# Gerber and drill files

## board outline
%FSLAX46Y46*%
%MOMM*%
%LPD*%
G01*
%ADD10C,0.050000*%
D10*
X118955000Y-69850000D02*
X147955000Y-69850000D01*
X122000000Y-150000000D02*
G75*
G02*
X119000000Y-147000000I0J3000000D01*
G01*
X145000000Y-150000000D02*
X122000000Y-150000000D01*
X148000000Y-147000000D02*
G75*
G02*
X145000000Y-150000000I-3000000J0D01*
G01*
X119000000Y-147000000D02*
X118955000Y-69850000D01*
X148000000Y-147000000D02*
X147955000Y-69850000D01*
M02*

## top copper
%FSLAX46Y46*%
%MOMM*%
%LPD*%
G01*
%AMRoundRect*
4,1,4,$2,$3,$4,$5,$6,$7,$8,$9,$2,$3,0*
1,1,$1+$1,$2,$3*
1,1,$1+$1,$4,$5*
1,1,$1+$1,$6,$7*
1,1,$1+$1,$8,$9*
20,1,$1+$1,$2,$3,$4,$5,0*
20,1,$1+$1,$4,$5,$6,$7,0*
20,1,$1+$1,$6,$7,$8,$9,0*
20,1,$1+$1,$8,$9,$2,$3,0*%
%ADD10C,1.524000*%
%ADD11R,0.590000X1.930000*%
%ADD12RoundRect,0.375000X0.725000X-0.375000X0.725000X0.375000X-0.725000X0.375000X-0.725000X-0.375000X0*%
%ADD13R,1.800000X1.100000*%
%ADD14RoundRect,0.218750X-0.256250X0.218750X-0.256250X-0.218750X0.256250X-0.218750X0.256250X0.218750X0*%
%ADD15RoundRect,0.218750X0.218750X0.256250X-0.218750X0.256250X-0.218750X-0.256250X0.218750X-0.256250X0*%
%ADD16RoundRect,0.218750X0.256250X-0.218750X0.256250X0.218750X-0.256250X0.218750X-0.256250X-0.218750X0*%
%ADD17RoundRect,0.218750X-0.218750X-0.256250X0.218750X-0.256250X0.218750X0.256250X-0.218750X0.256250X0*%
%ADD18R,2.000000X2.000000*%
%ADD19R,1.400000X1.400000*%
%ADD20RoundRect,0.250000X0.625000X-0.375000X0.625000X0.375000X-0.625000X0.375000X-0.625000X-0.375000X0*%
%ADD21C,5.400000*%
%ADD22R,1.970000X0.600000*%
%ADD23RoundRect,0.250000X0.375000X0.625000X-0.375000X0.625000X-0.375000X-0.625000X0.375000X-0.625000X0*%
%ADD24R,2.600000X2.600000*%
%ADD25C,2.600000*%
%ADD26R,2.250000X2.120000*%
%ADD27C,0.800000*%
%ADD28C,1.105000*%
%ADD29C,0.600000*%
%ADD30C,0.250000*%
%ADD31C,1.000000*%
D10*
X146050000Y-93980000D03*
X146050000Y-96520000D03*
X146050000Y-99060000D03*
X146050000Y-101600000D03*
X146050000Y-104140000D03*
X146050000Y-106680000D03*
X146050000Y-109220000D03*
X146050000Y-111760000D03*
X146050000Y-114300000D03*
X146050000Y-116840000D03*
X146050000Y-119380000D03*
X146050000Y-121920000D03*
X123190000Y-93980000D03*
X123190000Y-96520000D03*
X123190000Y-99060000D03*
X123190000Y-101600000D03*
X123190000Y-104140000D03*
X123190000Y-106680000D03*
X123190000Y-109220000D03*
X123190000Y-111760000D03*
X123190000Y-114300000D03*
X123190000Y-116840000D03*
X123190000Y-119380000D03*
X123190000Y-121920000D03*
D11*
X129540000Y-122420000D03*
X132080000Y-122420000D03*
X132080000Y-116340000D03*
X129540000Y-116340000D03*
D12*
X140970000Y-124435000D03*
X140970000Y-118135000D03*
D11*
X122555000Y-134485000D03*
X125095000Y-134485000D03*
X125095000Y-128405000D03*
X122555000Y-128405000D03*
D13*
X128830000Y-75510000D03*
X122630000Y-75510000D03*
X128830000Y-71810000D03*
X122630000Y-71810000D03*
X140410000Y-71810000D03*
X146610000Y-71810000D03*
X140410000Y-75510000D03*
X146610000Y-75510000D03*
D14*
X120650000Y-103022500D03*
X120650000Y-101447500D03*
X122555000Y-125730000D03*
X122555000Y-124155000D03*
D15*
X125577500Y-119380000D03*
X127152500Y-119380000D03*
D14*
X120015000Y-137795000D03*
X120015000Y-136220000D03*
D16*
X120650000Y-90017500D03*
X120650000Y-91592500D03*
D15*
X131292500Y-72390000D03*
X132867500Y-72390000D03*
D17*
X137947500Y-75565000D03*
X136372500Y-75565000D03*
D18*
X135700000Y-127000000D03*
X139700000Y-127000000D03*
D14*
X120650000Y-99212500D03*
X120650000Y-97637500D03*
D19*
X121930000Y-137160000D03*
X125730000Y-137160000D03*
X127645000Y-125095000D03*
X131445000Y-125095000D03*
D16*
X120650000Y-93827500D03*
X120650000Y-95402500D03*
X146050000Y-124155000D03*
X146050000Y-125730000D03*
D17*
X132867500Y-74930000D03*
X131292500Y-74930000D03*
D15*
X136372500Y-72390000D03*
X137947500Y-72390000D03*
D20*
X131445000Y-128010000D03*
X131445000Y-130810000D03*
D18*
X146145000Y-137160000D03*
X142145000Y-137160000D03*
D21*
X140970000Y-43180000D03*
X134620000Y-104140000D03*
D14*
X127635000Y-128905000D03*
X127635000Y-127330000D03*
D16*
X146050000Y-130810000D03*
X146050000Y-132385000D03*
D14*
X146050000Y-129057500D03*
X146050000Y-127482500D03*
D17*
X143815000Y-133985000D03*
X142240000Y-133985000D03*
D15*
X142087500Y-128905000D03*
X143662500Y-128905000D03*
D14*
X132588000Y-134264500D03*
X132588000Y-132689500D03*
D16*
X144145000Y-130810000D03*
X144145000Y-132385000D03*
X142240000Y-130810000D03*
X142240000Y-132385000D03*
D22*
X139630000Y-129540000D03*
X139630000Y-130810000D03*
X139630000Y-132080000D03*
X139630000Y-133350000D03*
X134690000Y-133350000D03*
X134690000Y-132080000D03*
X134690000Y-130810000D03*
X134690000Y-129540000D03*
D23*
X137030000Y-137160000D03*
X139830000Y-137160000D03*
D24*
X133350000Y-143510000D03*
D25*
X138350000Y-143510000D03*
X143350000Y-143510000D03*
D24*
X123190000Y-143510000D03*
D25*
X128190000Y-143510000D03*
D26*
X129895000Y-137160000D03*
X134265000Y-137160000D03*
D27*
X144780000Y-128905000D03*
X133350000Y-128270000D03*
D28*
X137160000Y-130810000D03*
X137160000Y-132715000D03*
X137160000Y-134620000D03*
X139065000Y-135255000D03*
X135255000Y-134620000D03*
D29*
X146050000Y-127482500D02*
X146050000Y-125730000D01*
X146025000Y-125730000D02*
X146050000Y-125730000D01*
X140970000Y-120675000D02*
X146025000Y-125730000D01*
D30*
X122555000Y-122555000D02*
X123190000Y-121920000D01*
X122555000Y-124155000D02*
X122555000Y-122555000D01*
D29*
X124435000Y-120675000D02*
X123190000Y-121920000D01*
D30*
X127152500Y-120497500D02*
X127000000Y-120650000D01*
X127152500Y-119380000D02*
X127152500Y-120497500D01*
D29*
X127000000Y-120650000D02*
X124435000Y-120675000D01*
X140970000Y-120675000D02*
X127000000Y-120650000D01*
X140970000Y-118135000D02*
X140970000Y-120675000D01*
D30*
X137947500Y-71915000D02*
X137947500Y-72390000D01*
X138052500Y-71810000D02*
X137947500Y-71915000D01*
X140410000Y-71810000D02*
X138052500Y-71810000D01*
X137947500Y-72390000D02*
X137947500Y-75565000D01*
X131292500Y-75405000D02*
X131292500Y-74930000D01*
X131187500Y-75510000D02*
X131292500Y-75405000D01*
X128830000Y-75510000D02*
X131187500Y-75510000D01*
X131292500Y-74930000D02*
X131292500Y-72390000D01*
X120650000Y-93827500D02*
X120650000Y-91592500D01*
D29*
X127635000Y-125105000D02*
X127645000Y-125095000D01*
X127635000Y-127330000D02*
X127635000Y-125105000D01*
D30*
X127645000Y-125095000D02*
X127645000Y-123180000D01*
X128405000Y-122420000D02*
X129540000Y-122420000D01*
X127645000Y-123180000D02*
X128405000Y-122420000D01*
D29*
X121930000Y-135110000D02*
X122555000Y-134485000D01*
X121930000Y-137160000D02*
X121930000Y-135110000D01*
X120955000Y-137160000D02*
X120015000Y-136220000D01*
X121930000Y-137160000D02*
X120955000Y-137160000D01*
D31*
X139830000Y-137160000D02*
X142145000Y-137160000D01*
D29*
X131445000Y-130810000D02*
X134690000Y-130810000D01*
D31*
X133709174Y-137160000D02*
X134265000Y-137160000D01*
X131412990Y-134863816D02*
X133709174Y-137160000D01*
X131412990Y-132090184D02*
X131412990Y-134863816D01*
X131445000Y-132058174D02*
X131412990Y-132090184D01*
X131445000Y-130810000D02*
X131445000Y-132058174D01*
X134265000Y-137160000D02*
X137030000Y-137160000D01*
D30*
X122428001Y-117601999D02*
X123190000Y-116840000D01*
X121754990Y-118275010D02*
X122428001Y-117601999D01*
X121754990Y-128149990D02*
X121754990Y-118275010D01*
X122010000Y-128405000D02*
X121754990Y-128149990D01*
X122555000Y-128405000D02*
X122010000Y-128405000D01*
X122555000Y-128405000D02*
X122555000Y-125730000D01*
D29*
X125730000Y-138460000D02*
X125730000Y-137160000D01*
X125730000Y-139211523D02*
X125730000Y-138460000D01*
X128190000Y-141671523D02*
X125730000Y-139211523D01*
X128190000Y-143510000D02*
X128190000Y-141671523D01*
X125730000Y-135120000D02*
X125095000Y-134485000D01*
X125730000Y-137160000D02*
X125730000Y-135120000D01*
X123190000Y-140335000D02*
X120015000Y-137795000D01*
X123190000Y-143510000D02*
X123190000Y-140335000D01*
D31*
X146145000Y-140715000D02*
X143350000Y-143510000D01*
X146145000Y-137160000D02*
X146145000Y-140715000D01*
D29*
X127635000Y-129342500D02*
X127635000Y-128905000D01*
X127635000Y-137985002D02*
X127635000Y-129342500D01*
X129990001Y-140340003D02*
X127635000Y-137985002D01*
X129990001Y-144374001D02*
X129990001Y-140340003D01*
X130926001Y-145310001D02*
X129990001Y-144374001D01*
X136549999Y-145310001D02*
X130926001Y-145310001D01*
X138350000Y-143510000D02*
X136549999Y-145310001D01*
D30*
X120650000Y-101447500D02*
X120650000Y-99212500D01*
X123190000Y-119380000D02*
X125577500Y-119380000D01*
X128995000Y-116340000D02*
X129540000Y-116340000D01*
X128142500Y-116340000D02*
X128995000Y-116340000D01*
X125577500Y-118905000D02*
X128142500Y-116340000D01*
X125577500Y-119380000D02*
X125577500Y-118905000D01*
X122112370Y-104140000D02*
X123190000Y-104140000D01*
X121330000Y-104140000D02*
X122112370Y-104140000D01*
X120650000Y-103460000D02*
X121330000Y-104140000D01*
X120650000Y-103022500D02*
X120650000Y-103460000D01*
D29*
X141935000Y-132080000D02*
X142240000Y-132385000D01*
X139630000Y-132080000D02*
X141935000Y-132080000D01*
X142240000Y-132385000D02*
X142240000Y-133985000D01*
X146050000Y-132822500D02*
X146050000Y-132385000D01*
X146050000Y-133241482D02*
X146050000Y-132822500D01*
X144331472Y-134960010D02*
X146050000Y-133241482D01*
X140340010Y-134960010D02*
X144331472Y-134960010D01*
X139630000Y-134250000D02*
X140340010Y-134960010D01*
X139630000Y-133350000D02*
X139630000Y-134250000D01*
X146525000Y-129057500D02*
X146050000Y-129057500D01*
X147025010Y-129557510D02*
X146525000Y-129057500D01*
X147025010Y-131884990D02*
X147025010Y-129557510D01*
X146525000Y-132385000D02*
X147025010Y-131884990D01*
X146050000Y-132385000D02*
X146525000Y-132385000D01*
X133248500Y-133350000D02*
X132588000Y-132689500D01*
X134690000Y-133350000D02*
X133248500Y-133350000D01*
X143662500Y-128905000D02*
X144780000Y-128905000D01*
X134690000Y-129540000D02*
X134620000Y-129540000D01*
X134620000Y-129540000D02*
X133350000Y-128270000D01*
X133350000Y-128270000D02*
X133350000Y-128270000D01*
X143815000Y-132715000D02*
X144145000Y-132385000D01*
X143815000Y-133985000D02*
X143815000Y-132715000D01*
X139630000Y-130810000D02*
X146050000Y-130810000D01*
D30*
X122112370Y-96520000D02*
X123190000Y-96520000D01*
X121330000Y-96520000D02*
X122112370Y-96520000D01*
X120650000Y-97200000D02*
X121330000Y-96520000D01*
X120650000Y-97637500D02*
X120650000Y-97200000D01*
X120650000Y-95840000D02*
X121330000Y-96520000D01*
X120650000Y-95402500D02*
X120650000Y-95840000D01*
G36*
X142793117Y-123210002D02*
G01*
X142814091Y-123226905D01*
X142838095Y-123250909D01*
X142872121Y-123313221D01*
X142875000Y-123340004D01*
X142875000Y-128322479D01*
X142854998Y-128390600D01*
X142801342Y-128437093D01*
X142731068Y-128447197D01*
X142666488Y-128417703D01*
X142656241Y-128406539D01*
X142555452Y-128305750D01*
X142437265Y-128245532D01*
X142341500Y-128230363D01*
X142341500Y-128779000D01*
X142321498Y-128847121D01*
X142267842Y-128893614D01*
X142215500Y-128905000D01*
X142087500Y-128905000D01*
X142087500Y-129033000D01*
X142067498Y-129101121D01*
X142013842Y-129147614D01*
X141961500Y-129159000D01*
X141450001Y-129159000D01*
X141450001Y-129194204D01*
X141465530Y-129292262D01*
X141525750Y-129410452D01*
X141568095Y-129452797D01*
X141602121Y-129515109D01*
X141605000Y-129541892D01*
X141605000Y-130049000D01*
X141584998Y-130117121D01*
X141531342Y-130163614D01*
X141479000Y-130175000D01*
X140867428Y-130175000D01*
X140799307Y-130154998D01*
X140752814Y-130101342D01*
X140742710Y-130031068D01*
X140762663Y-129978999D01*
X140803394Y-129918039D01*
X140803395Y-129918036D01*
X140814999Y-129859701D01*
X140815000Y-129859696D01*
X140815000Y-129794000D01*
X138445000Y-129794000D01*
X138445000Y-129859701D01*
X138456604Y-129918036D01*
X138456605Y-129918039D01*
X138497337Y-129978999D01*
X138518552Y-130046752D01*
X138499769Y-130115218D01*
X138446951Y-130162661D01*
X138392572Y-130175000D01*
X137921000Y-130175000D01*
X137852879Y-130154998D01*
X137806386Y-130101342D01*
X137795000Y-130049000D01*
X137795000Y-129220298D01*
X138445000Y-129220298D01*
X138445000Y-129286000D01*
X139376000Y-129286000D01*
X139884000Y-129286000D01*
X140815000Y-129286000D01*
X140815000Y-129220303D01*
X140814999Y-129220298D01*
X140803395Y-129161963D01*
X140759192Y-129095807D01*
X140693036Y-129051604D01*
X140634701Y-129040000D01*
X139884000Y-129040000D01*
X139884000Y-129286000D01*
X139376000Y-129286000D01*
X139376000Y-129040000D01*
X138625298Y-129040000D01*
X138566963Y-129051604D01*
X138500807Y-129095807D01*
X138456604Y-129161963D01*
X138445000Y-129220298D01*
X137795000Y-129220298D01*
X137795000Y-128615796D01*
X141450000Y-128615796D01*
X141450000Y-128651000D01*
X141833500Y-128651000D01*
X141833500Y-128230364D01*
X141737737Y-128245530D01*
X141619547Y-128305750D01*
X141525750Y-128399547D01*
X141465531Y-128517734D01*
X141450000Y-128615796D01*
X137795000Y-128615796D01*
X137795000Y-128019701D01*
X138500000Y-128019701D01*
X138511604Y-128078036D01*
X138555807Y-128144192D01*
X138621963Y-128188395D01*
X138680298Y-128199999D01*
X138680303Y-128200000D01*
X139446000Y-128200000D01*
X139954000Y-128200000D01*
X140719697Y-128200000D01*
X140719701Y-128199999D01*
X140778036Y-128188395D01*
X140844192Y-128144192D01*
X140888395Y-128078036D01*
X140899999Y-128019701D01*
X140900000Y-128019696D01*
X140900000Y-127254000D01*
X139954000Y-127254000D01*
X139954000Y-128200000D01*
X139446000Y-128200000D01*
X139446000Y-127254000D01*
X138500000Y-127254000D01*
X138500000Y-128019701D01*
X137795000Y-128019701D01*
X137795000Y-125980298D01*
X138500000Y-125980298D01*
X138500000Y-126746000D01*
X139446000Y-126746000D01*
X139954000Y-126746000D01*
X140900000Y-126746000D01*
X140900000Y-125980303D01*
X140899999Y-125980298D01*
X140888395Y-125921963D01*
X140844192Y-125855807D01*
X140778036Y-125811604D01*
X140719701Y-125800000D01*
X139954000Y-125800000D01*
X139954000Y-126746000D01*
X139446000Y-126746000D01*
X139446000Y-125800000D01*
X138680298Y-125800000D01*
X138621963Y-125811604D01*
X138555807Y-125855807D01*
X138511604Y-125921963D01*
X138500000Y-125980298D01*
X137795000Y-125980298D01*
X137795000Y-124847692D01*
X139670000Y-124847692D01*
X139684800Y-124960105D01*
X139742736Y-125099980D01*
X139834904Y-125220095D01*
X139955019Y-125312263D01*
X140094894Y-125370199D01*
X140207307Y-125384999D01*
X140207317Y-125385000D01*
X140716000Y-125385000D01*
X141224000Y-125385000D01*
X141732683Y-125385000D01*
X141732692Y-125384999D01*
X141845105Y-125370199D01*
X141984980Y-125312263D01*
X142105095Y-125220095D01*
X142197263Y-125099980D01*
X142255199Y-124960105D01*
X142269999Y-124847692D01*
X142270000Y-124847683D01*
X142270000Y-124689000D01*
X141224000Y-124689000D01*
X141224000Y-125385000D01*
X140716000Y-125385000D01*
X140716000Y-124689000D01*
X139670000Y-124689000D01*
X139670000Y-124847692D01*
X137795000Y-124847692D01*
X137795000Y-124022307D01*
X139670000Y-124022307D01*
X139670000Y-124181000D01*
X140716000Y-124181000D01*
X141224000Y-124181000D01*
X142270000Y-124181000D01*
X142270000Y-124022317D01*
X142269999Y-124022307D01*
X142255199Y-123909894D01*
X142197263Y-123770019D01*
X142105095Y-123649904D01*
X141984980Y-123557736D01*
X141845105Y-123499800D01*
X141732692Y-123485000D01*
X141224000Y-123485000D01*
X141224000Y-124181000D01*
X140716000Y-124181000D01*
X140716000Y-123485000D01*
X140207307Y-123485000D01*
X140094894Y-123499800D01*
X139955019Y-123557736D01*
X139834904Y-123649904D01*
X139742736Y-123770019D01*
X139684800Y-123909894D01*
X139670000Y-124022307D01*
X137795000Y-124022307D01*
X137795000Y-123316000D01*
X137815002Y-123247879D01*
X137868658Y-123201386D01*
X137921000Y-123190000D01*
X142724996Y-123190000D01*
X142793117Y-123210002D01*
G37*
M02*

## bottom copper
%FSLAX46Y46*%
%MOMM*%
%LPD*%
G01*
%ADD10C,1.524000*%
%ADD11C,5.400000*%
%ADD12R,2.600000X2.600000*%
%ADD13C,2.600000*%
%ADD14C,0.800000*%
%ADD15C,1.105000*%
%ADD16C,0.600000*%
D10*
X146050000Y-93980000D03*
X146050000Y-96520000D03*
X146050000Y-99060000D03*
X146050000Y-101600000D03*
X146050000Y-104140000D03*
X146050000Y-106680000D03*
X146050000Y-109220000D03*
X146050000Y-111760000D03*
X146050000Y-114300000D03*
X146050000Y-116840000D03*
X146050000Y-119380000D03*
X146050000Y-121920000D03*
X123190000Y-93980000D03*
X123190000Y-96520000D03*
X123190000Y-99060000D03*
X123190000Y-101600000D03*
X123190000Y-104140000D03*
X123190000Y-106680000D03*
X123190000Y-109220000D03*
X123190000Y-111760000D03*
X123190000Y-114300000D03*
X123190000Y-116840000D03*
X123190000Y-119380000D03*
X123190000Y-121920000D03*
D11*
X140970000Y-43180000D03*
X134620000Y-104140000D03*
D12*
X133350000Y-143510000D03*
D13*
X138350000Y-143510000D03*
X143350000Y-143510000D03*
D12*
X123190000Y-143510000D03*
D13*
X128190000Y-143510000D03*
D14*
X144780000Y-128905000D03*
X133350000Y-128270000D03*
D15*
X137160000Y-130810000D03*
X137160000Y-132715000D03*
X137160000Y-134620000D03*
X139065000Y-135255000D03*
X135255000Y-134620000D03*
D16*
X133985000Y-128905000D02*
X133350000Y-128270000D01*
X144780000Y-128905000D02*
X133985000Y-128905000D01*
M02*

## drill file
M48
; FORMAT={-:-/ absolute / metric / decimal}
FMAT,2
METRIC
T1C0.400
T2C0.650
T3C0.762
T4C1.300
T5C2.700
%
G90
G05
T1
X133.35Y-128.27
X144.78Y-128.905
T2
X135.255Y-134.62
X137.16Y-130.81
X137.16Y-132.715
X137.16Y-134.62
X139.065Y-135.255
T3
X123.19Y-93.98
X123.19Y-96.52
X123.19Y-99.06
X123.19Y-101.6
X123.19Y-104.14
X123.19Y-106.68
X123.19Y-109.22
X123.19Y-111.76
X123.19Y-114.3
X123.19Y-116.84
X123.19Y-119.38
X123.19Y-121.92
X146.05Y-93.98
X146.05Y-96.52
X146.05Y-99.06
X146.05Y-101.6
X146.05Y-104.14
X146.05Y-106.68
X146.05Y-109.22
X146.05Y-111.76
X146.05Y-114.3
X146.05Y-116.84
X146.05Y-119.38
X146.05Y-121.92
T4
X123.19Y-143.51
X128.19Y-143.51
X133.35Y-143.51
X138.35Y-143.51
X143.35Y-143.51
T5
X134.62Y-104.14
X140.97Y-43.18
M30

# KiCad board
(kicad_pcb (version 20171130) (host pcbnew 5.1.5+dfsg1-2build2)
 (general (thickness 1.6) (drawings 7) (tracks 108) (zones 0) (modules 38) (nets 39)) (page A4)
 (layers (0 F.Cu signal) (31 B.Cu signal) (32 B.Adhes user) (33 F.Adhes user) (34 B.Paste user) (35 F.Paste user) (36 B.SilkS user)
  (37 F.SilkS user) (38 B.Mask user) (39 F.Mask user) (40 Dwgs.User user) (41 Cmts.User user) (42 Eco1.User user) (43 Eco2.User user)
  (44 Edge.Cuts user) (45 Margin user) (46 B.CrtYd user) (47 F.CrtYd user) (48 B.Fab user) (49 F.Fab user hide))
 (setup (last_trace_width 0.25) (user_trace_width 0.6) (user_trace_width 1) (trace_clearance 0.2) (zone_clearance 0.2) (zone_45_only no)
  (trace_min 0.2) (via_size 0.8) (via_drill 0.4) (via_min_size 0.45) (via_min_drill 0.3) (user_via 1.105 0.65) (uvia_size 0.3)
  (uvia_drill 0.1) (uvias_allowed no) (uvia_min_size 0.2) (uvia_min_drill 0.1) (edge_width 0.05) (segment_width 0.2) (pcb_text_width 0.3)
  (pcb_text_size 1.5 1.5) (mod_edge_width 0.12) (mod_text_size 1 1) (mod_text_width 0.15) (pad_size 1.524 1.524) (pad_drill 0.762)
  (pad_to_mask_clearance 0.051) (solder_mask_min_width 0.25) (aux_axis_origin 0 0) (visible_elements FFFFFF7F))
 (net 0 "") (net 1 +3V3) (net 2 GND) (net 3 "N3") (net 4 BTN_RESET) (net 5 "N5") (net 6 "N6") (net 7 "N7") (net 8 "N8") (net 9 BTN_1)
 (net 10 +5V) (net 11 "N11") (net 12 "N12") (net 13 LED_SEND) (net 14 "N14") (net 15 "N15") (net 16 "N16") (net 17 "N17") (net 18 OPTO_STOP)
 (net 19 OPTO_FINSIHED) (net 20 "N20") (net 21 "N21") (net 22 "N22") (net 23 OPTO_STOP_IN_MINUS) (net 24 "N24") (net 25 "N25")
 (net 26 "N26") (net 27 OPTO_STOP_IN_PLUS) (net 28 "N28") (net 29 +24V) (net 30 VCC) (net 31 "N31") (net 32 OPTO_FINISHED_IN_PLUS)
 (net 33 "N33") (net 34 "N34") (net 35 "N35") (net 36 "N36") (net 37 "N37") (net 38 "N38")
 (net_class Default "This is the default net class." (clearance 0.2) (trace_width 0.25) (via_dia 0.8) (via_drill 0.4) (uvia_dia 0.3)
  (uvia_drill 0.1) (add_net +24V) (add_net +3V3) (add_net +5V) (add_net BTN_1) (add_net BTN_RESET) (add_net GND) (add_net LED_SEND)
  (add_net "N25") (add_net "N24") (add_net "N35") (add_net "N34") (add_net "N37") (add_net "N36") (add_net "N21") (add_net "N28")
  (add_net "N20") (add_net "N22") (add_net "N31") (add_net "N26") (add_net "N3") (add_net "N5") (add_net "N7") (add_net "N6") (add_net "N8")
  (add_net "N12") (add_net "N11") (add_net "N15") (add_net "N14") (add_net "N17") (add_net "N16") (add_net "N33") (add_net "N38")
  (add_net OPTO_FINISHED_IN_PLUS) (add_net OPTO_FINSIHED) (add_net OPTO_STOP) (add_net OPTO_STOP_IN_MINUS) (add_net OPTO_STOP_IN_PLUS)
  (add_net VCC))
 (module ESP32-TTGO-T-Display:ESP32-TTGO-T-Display (layer F.Cu) (at 134.62 104.14 180)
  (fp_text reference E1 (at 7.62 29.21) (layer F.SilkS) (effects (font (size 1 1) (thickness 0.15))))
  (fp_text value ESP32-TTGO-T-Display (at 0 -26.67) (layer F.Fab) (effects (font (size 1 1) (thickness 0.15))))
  (pad 3V3-1 thru_hole circle (at -11.43 10.16 180) (size 1.524 1.524) (drill 0.762) (layers *.Cu *.Mask) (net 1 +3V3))
  (pad G4 thru_hole circle (at -11.43 7.62 180) (size 1.524 1.524) (drill 0.762) (layers *.Cu *.Mask) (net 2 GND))
  (pad G3 thru_hole circle (at -11.43 5.08 180) (size 1.524 1.524) (drill 0.762) (layers *.Cu *.Mask) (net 2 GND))
  (pad 12 thru_hole circle (at -11.43 2.54 180) (size 1.524 1.524) (drill 0.762) (layers *.Cu *.Mask) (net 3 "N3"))
  (pad 13 thru_hole circle (at -11.43 0 180) (size 1.524 1.524) (drill 0.762) (layers *.Cu *.Mask) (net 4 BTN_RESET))
  (pad 15 thru_hole circle (at -11.43 -2.54 180) (size 1.524 1.524) (drill 0.762) (layers *.Cu *.Mask) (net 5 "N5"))
  (pad 2 thru_hole circle (at -11.43 -5.08 180) (size 1.524 1.524) (drill 0.762) (layers *.Cu *.Mask) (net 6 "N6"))
  (pad 17 thru_hole circle (at -11.43 -7.62 180) (size 1.524 1.524) (drill 0.762) (layers *.Cu *.Mask) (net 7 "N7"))
  (pad 22 thru_hole circle (at -11.43 -10.16 180) (size 1.524 1.524) (drill 0.762) (layers *.Cu *.Mask) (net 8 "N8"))
  (pad 21 thru_hole circle (at -11.43 -12.7 180) (size 1.524 1.524) (drill 0.762) (layers *.Cu *.Mask) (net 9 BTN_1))
  (pad G2 thru_hole circle (at -11.43 -15.24 180) (size 1.524 1.524) (drill 0.762) (layers *.Cu *.Mask) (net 2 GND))
  (pad G1 thru_hole circle (at -11.43 -17.78 180) (size 1.524 1.524) (drill 0.762) (layers *.Cu *.Mask) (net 2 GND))
  (pad 5V thru_hole circle (at 11.43 10.16 180) (size 1.524 1.524) (drill 0.762) (layers *.Cu *.Mask) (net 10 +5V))
  (pad G5 thru_hole circle (at 11.43 7.62 180) (size 1.524 1.524) (drill 0.762) (layers *.Cu *.Mask) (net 2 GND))
  (pad 27 thru_hole circle (at 11.43 5.08 180) (size 1.524 1.524) (drill 0.762) (layers *.Cu *.Mask) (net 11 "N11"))
  (pad 26 thru_hole circle (at 11.43 2.54 180) (size 1.524 1.524) (drill 0.762) (layers *.Cu *.Mask) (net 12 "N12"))
  (pad 25 thru_hole circle (at 11.43 0 180) (size 1.524 1.524) (drill 0.762) (layers *.Cu *.Mask) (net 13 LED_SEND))
  (pad 33 thru_hole circle (at 11.43 -2.54 180) (size 1.524 1.524) (drill 0.762) (layers *.Cu *.Mask) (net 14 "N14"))
  (pad 32 thru_hole circle (at 11.43 -5.08 180) (size 1.524 1.524) (drill 0.762) (layers *.Cu *.Mask) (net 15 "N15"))
  (pad 39 thru_hole circle (at 11.43 -7.62 180) (size 1.524 1.524) (drill 0.762) (layers *.Cu *.Mask) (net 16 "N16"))
  (pad 38 thru_hole circle (at 11.43 -10.16 180) (size 1.524 1.524) (drill 0.762) (layers *.Cu *.Mask) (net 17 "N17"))
  (pad 37 thru_hole circle (at 11.43 -12.7 180) (size 1.524 1.524) (drill 0.762) (layers *.Cu *.Mask) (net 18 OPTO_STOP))
  (pad 36 thru_hole circle (at 11.43 -15.24 180) (size 1.524 1.524) (drill 0.762) (layers *.Cu *.Mask) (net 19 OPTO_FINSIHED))
  (pad 3V3-2 thru_hole circle (at 11.43 -17.78 180) (size 1.524 1.524) (drill 0.762) (layers *.Cu *.Mask) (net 1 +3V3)))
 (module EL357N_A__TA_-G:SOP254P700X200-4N (layer F.Cu) (at 130.81 119.38 90)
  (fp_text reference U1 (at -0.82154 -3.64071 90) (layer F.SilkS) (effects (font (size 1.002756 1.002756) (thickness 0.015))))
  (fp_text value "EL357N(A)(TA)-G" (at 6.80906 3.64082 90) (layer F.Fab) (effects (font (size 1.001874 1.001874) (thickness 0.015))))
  (pad 1 smd rect (at -3.04 -1.27 90) (size 1.93 0.59) (layers F.Cu F.Paste F.Mask) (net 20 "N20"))
  (pad 2 smd rect (at -3.04 1.27 90) (size 1.93 0.59) (layers F.Cu F.Paste F.Mask) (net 2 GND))
  (pad 3 smd rect (at 3.04 1.27 90) (size 1.93 0.59) (layers F.Cu F.Paste F.Mask) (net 2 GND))
  (pad 4 smd rect (at 3.04 -1.27 90) (size 1.93 0.59) (layers F.Cu F.Paste F.Mask) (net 19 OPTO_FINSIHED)))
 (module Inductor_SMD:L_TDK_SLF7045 (layer F.Cu) (at 140.97 121.285 90)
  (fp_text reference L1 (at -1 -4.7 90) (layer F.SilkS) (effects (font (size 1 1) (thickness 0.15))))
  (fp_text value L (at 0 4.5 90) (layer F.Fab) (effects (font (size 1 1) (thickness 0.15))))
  (pad 1 smd roundrect (at -3.15 0 90) (size 1.5 2.2) (layers F.Cu F.Paste F.Mask) (roundrect_rratio 0.25) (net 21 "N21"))
  (pad 2 smd roundrect (at 3.15 0 90) (size 1.5 2.2) (layers F.Cu F.Paste F.Mask) (roundrect_rratio 0.25) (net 1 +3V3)))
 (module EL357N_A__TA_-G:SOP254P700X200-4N (layer F.Cu) (at 123.825 131.445 90)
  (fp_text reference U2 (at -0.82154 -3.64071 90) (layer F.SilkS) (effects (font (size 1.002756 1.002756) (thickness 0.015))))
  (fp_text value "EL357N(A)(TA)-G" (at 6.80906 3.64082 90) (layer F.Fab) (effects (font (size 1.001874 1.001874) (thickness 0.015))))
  (pad 1 smd rect (at -3.04 -1.27 90) (size 1.93 0.59) (layers F.Cu F.Paste F.Mask) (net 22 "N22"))
  (pad 2 smd rect (at -3.04 1.27 90) (size 1.93 0.59) (layers F.Cu F.Paste F.Mask) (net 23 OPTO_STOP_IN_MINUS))
  (pad 3 smd rect (at 3.04 1.27 90) (size 1.93 0.59) (layers F.Cu F.Paste F.Mask) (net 2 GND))
  (pad 4 smd rect (at 3.04 -1.27 90) (size 1.93 0.59) (layers F.Cu F.Paste F.Mask) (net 18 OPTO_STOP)))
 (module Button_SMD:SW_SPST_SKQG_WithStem (layer F.Cu) (at 125.73 73.66 180)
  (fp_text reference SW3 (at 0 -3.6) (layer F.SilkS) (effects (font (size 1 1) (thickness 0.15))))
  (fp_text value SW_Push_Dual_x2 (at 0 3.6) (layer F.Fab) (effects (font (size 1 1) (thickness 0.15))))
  (pad 1 smd rect (at -3.1 -1.85 180) (size 1.8 1.1) (layers F.Cu F.Paste F.Mask) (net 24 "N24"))
  (pad 1 smd rect (at 3.1 -1.85 180) (size 1.8 1.1) (layers F.Cu F.Paste F.Mask) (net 24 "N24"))
  (pad 2 smd rect (at -3.1 1.85 180) (size 1.8 1.1) (layers F.Cu F.Paste F.Mask) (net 2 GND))
  (pad 2 smd rect (at 3.1 1.85 180) (size 1.8 1.1) (layers F.Cu F.Paste F.Mask) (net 2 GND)))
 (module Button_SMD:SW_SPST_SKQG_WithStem (layer F.Cu) (at 143.51 73.66)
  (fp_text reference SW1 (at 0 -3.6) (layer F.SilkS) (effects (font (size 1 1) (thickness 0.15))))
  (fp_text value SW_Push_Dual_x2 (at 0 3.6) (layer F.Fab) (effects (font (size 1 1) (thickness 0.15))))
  (pad 1 smd rect (at -3.1 -1.85) (size 1.8 1.1) (layers F.Cu F.Paste F.Mask) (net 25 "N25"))
  (pad 1 smd rect (at 3.1 -1.85) (size 1.8 1.1) (layers F.Cu F.Paste F.Mask) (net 25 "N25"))
  (pad 2 smd rect (at -3.1 1.85) (size 1.8 1.1) (layers F.Cu F.Paste F.Mask) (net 2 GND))
  (pad 2 smd rect (at 3.1 1.85) (size 1.8 1.1) (layers F.Cu F.Paste F.Mask) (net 2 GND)))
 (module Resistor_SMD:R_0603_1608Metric (layer F.Cu) (at 120.65 102.235 270)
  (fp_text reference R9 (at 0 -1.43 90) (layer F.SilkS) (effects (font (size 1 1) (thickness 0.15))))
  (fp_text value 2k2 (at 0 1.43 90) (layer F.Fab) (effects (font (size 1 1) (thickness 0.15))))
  (pad 2 smd roundrect (at 0.7875 0 270) (size 0.875 0.95) (layers F.Cu F.Paste F.Mask) (roundrect_rratio 0.25) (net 13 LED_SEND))
  (pad 1 smd roundrect (at -0.7875 0 270) (size 0.875 0.95) (layers F.Cu F.Paste F.Mask) (roundrect_rratio 0.25) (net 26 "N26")))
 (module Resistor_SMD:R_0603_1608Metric (layer F.Cu) (at 122.555 124.9425 270)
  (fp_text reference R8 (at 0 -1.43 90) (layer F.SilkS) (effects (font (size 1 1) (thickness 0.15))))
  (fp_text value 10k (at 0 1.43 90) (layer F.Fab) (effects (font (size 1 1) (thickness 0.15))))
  (pad 2 smd roundrect (at 0.7875 0 270) (size 0.875 0.95) (layers F.Cu F.Paste F.Mask) (roundrect_rratio 0.25) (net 18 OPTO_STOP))
  (pad 1 smd roundrect (at -0.7875 0 270) (size 0.875 0.95) (layers F.Cu F.Paste F.Mask) (roundrect_rratio 0.25) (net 1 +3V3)))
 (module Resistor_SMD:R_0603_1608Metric (layer F.Cu) (at 126.365 119.38 180)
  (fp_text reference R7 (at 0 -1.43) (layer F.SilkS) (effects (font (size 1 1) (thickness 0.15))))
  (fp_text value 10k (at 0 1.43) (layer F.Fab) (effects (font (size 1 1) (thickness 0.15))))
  (pad 2 smd roundrect (at 0.7875 0 180) (size 0.875 0.95) (layers F.Cu F.Paste F.Mask) (roundrect_rratio 0.25) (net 19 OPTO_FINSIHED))
  (pad 1 smd roundrect (at -0.7875 0 180) (size 0.875 0.95) (layers F.Cu F.Paste F.Mask) (roundrect_rratio 0.25) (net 1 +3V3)))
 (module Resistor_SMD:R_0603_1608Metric (layer F.Cu) (at 120.015 137.0075 270)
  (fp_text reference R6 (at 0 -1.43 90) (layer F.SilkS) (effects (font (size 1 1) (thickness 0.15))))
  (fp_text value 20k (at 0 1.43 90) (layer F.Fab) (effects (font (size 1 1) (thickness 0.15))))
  (pad 2 smd roundrect (at 0.7875 0 270) (size 0.875 0.95) (layers F.Cu F.Paste F.Mask) (roundrect_rratio 0.25) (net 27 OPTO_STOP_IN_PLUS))
  (pad 1 smd roundrect (at -0.7875 0 270) (size 0.875 0.95) (layers F.Cu F.Paste F.Mask) (roundrect_rratio 0.25) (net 22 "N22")))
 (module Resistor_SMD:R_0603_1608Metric (layer F.Cu) (at 120.65 90.805 90)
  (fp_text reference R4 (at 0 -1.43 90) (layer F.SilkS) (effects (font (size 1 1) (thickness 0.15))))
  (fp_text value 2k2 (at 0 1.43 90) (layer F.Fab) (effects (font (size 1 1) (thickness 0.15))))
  (pad 2 smd roundrect (at 0.7875 0 90) (size 0.875 0.95) (layers F.Cu F.Paste F.Mask) (roundrect_rratio 0.25) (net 1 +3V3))
  (pad 1 smd roundrect (at -0.7875 0 90) (size 0.875 0.95) (layers F.Cu F.Paste F.Mask) (roundrect_rratio 0.25) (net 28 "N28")))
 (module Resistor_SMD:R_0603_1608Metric (layer F.Cu) (at 132.08 72.39 180)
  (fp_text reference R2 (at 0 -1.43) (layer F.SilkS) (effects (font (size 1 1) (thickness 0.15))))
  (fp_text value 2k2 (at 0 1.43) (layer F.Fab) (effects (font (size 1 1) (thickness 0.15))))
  (pad 2 smd roundrect (at 0.7875 0 180) (size 0.875 0.95) (layers F.Cu F.Paste F.Mask) (roundrect_rratio 0.25) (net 24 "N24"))
  (pad 1 smd roundrect (at -0.7875 0 180) (size 0.875 0.95) (layers F.Cu F.Paste F.Mask) (roundrect_rratio 0.25) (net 9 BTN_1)))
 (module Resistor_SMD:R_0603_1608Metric (layer F.Cu) (at 137.16 75.565)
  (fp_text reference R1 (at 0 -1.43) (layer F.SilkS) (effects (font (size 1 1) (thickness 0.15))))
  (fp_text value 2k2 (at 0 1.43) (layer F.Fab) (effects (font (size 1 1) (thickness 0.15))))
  (pad 2 smd roundrect (at 0.7875 0) (size 0.875 0.95) (layers F.Cu F.Paste F.Mask) (roundrect_rratio 0.25) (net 25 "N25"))
  (pad 1 smd roundrect (at -0.7875 0) (size 0.875 0.95) (layers F.Cu F.Paste F.Mask) (roundrect_rratio 0.25) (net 4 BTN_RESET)))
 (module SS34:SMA (layer F.Cu) (at 137.7 127 180)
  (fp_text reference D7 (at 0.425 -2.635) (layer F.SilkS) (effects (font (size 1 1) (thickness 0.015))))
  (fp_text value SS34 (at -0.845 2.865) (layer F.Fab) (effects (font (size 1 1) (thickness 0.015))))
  (pad A smd rect (at 2 0 180) (size 2 2) (layers F.Cu F.Paste F.Mask) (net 2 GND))
  (pad C smd rect (at -2 0 180) (size 2 2) (layers F.Cu F.Paste F.Mask) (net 21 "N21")))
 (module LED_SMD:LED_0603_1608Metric (layer F.Cu) (at 120.65 98.425 270)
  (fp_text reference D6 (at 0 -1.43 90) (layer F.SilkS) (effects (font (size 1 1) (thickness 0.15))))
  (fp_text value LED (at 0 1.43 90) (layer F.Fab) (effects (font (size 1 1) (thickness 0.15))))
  (pad 2 smd roundrect (at 0.7875 0 270) (size 0.875 0.95) (layers F.Cu F.Paste F.Mask) (roundrect_rratio 0.25) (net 26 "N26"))
  (pad 1 smd roundrect (at -0.7875 0 270) (size 0.875 0.95) (layers F.Cu F.Paste F.Mask) (roundrect_rratio 0.25) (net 2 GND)))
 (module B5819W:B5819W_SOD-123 (layer F.Cu) (at 123.83 137.16)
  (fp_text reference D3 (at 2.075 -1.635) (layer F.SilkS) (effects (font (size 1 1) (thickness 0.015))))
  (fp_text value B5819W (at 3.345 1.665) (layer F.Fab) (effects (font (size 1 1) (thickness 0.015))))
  (pad C smd rect (at -1.9 0) (size 1.4 1.4) (layers F.Cu F.Paste F.Mask) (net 22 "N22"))
  (pad A smd rect (at 1.9 0) (size 1.4 1.4) (layers F.Cu F.Paste F.Mask) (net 23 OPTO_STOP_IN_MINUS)))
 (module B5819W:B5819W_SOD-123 (layer F.Cu) (at 129.545 125.095)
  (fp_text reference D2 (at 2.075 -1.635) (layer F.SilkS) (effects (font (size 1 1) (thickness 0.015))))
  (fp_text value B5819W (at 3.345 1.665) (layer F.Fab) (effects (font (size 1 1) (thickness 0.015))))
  (pad C smd rect (at -1.9 0) (size 1.4 1.4) (layers F.Cu F.Paste F.Mask) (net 20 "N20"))
  (pad A smd rect (at 1.9 0) (size 1.4 1.4) (layers F.Cu F.Paste F.Mask) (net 2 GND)))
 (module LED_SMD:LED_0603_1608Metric (layer F.Cu) (at 120.65 94.615 90)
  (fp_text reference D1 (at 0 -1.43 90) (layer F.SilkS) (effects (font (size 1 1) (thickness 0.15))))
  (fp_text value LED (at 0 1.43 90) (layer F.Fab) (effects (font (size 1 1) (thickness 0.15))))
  (pad 2 smd roundrect (at 0.7875 0 90) (size 0.875 0.95) (layers F.Cu F.Paste F.Mask) (roundrect_rratio 0.25) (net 28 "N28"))
  (pad 1 smd roundrect (at -0.7875 0 90) (size 0.875 0.95) (layers F.Cu F.Paste F.Mask) (roundrect_rratio 0.25) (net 2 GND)))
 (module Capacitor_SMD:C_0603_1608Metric (layer F.Cu) (at 146.05 124.9425 90)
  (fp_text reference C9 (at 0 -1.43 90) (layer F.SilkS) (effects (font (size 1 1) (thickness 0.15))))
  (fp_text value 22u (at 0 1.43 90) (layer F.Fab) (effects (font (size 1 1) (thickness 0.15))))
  (pad 2 smd roundrect (at 0.7875 0 90) (size 0.875 0.95) (layers F.Cu F.Paste F.Mask) (roundrect_rratio 0.25) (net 2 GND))
  (pad 1 smd roundrect (at -0.7875 0 90) (size 0.875 0.95) (layers F.Cu F.Paste F.Mask) (roundrect_rratio 0.25) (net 1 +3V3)))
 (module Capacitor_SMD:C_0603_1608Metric (layer F.Cu) (at 132.08 74.93)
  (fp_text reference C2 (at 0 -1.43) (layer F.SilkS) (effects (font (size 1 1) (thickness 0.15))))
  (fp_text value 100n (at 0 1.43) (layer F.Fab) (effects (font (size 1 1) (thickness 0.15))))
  (pad 2 smd roundrect (at 0.7875 0) (size 0.875 0.95) (layers F.Cu F.Paste F.Mask) (roundrect_rratio 0.25) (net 2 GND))
  (pad 1 smd roundrect (at -0.7875 0) (size 0.875 0.95) (layers F.Cu F.Paste F.Mask) (roundrect_rratio 0.25) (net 24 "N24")))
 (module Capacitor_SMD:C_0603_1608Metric (layer F.Cu) (at 137.16 72.39 180)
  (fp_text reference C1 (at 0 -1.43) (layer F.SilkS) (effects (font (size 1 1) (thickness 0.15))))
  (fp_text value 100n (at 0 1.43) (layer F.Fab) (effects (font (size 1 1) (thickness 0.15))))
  (pad 2 smd roundrect (at 0.7875 0 180) (size 0.875 0.95) (layers F.Cu F.Paste F.Mask) (roundrect_rratio 0.25) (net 2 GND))
  (pad 1 smd roundrect (at -0.7875 0 180) (size 0.875 0.95) (layers F.Cu F.Paste F.Mask) (roundrect_rratio 0.25) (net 25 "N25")))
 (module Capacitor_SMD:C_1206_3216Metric (layer F.Cu) (at 131.445 129.41 90)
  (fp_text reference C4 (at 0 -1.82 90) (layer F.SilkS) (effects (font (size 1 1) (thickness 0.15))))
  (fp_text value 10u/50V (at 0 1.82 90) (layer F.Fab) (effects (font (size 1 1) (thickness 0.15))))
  (pad 2 smd roundrect (at 1.4 0 90) (size 1.25 1.75) (layers F.Cu F.Paste F.Mask) (roundrect_rratio 0.2) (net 2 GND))
  (pad 1 smd roundrect (at -1.4 0 90) (size 1.25 1.75) (layers F.Cu F.Paste F.Mask) (roundrect_rratio 0.2) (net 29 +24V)))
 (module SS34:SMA (layer F.Cu) (at 144.145 137.16)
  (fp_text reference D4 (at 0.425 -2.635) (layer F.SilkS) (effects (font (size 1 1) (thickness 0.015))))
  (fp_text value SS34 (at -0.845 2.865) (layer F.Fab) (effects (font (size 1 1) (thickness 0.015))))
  (pad A smd rect (at 2 0) (size 2 2) (layers F.Cu F.Paste F.Mask) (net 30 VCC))
  (pad C smd rect (at -2 0) (size 2 2) (layers F.Cu F.Paste F.Mask) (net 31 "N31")))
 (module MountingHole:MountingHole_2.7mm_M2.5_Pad (layer F.Cu) (at 140.97 43.18)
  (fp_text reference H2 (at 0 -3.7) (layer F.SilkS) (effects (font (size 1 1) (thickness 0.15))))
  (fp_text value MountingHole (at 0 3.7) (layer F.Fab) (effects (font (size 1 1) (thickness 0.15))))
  (pad 1 thru_hole circle (at 0 0) (size 5.4 5.4) (drill 2.7) (layers *.Cu *.Mask)))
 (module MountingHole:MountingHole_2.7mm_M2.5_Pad (layer F.Cu) (at 134.62 104.14)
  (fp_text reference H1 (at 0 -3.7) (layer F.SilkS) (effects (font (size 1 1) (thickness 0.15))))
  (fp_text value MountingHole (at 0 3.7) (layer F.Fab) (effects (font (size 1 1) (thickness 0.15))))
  (pad 1 thru_hole circle (at 0 0) (size 5.4 5.4) (drill 2.7) (layers *.Cu *.Mask)))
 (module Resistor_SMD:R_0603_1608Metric (layer F.Cu) (at 127.635 128.1175 270)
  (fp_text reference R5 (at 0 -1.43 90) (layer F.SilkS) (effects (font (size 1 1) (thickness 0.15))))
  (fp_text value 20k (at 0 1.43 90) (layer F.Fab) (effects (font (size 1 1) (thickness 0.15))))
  (pad 2 smd roundrect (at 0.7875 0 270) (size 0.875 0.95) (layers F.Cu F.Paste F.Mask) (roundrect_rratio 0.25)
   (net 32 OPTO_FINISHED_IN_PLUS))
  (pad 1 smd roundrect (at -0.7875 0 270) (size 0.875 0.95) (layers F.Cu F.Paste F.Mask) (roundrect_rratio 0.25) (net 20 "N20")))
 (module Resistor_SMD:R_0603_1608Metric (layer F.Cu) (at 146.05 131.5975 90)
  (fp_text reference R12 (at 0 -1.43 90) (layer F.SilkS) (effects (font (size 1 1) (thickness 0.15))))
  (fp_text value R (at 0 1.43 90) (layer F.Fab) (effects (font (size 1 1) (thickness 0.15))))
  (pad 2 smd roundrect (at 0.7875 0 90) (size 0.875 0.95) (layers F.Cu F.Paste F.Mask) (roundrect_rratio 0.25) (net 2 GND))
  (pad 1 smd roundrect (at -0.7875 0 90) (size 0.875 0.95) (layers F.Cu F.Paste F.Mask) (roundrect_rratio 0.25) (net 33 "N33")))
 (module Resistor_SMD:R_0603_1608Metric (layer F.Cu) (at 146.05 128.27 270)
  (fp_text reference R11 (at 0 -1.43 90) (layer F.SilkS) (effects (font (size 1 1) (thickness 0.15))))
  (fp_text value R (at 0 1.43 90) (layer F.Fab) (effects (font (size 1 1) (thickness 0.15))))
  (pad 2 smd roundrect (at 0.7875 0 270) (size 0.875 0.95) (layers F.Cu F.Paste F.Mask) (roundrect_rratio 0.25) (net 33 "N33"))
  (pad 1 smd roundrect (at -0.7875 0 270) (size 0.875 0.95) (layers F.Cu F.Paste F.Mask) (roundrect_rratio 0.25) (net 1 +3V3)))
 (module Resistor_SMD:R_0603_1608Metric (layer F.Cu) (at 143.0275 133.985)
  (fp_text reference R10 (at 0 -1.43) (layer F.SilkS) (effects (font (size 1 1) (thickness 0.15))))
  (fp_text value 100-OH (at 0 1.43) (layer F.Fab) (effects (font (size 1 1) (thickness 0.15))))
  (pad 2 smd roundrect (at 0.7875 0) (size 0.875 0.95) (layers F.Cu F.Paste F.Mask) (roundrect_rratio 0.25) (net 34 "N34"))
  (pad 1 smd roundrect (at -0.7875 0) (size 0.875 0.95) (layers F.Cu F.Paste F.Mask) (roundrect_rratio 0.25) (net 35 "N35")))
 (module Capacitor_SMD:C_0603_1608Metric (layer F.Cu) (at 142.875 128.905 180)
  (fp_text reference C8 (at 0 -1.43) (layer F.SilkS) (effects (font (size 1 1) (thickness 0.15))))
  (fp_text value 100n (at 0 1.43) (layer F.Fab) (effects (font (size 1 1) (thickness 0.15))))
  (pad 2 smd roundrect (at 0.7875 0 180) (size 0.875 0.95) (layers F.Cu F.Paste F.Mask) (roundrect_rratio 0.25) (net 21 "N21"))
  (pad 1 smd roundrect (at -0.7875 0 180) (size 0.875 0.95) (layers F.Cu F.Paste F.Mask) (roundrect_rratio 0.25) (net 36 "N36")))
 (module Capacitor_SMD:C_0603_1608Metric (layer F.Cu) (at 132.588 133.477 270)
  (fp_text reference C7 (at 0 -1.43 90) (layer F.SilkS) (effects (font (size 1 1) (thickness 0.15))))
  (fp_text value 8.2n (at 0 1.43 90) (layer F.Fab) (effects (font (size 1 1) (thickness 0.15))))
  (pad 2 smd roundrect (at 0.7875 0 270) (size 0.875 0.95) (layers F.Cu F.Paste F.Mask) (roundrect_rratio 0.25) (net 2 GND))
  (pad 1 smd roundrect (at -0.7875 0 270) (size 0.875 0.95) (layers F.Cu F.Paste F.Mask) (roundrect_rratio 0.25) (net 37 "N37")))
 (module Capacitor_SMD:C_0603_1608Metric (layer F.Cu) (at 144.145 131.5975 90)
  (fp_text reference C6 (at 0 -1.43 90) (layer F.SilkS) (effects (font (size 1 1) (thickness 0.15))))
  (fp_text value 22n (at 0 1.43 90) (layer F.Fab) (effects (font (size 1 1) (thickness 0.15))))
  (pad 2 smd roundrect (at 0.7875 0 90) (size 0.875 0.95) (layers F.Cu F.Paste F.Mask) (roundrect_rratio 0.25) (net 2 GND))
  (pad 1 smd roundrect (at -0.7875 0 90) (size 0.875 0.95) (layers F.Cu F.Paste F.Mask) (roundrect_rratio 0.25) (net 34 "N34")))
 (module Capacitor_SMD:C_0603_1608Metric (layer F.Cu) (at 142.24 131.5975 90)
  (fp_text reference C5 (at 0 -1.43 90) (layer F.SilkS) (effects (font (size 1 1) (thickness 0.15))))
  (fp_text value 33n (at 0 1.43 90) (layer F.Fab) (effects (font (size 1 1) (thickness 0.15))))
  (pad 2 smd roundrect (at 0.7875 0 90) (size 0.875 0.95) (layers F.Cu F.Paste F.Mask) (roundrect_rratio 0.25) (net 2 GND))
  (pad 1 smd roundrect (at -0.7875 0 90) (size 0.875 0.95) (layers F.Cu F.Paste F.Mask) (roundrect_rratio 0.25) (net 35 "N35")))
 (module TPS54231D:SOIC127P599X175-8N (layer F.Cu) (at 137.16 131.445)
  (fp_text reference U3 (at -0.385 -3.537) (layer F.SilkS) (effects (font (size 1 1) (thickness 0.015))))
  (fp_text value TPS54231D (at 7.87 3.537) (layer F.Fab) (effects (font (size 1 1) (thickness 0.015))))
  (pad 8 smd rect (at 2.47 -1.905) (size 1.97 0.6) (layers F.Cu F.Paste F.Mask) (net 21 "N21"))
  (pad 7 smd rect (at 2.47 -0.635) (size 1.97 0.6) (layers F.Cu F.Paste F.Mask) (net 2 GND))
  (pad 6 smd rect (at 2.47 0.635) (size 1.97 0.6) (layers F.Cu F.Paste F.Mask) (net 35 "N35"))
  (pad 5 smd rect (at 2.47 1.905) (size 1.97 0.6) (layers F.Cu F.Paste F.Mask) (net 33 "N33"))
  (pad 4 smd rect (at -2.47 1.905) (size 1.97 0.6) (layers F.Cu F.Paste F.Mask) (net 37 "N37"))
  (pad 3 smd rect (at -2.47 0.635) (size 1.97 0.6) (layers F.Cu F.Paste F.Mask) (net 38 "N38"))
  (pad 2 smd rect (at -2.47 -0.635) (size 1.97 0.6) (layers F.Cu F.Paste F.Mask) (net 29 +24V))
  (pad 1 smd rect (at -2.47 -1.905) (size 1.97 0.6) (layers F.Cu F.Paste F.Mask) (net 36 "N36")))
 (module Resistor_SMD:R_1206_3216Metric (layer F.Cu) (at 138.43 137.16 180)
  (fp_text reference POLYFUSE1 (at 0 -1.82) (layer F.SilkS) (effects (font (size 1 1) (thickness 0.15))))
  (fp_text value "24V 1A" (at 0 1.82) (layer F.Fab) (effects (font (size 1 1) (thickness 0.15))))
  (pad 2 smd roundrect (at 1.4 0 180) (size 1.25 1.75) (layers F.Cu F.Paste F.Mask) (roundrect_rratio 0.2) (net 29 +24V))
  (pad 1 smd roundrect (at -1.4 0 180) (size 1.25 1.75) (layers F.Cu F.Paste F.Mask) (roundrect_rratio 0.2) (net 31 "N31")))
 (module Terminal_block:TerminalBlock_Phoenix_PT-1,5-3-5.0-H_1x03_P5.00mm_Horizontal (layer F.Cu) (at 133.35 143.51)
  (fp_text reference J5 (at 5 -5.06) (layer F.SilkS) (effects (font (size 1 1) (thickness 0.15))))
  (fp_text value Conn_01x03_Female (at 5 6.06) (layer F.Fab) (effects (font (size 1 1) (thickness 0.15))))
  (pad 1 thru_hole rect (at 0 0) (size 2.6 2.6) (drill 1.3) (layers *.Cu *.Mask) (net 2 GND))
  (pad 2 thru_hole circle (at 5 0) (size 2.6 2.6) (drill 1.3) (layers *.Cu *.Mask) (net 32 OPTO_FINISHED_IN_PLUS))
  (pad 3 thru_hole circle (at 10 0) (size 2.6 2.6) (drill 1.3) (layers *.Cu *.Mask) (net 30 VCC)))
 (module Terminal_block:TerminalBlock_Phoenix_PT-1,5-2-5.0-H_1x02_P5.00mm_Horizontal (layer F.Cu) (at 123.19 143.51)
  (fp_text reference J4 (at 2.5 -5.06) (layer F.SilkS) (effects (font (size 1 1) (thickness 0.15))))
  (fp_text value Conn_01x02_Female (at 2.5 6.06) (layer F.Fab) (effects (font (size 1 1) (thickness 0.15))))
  (pad 1 thru_hole rect (at 0 0) (size 2.6 2.6) (drill 1.3) (layers *.Cu *.Mask) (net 27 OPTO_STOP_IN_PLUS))
  (pad 2 thru_hole circle (at 5 0) (size 2.6 2.6) (drill 1.3) (layers *.Cu *.Mask) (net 23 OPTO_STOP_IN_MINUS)))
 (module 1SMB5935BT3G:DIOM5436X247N (layer F.Cu) (at 132.08 137.16 180)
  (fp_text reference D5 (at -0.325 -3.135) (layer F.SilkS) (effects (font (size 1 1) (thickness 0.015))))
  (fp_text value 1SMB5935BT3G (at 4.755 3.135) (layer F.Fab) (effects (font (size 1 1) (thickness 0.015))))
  (pad A smd rect (at 2.185 0 180) (size 2.25 2.12) (layers F.Cu F.Paste F.Mask) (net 2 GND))
  (pad C smd rect (at -2.185 0 180) (size 2.25 2.12) (layers F.Cu F.Paste F.Mask) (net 29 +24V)))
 (gr_line (start 118.955 69.85) (end 147.955 69.85) (layer Edge.Cuts) (width 0.05))
 (gr_arc (start 122 147) (end 119 147) (angle -90) (layer Edge.Cuts) (width 0.05))
 (gr_line (start 145 150) (end 122 150) (layer Edge.Cuts) (width 0.05))
 (gr_arc (start 145 147) (end 145 150) (angle -90) (layer Edge.Cuts) (width 0.05))
 (gr_line (start 119 147) (end 118.955 69.85) (layer Edge.Cuts) (width 0.05))
 (gr_line (start 148 147) (end 147.955 69.85) (layer Edge.Cuts) (width 0.05))
 (segment (start 146.05 127.4825) (end 146.05 125.73) (width 0.6) (layer F.Cu) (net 1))
 (segment (start 146.025 125.73) (end 146.05 125.73) (width 0.6) (layer F.Cu) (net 1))
 (segment (start 140.97 120.675) (end 146.025 125.73) (width 0.6) (layer F.Cu) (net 1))
 (segment (start 122.555 122.555) (end 123.19 121.92) (width 0.25) (layer F.Cu) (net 1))
 (segment (start 122.555 124.155) (end 122.555 122.555) (width 0.25) (layer F.Cu) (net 1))
 (segment (start 124.435 120.675) (end 123.19 121.92) (width 0.6) (layer F.Cu) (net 1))
 (segment (start 127.1525 120.4975) (end 127 120.65) (width 0.25) (layer F.Cu) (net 1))
 (segment (start 127.1525 119.38) (end 127.1525 120.4975) (width 0.25) (layer F.Cu) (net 1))
 (segment (start 127 120.65) (end 124.435 120.675) (width 0.6) (layer F.Cu) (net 1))
 (segment (start 140.97 120.675) (end 127 120.65) (width 0.6) (layer F.Cu) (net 1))
 (segment (start 140.97 118.135) (end 140.97 120.675) (width 0.6) (layer F.Cu) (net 1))
 (segment (start 137.9475 71.915) (end 137.9475 72.39) (width 0.25) (layer F.Cu) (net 25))
 (segment (start 138.0525 71.81) (end 137.9475 71.915) (width 0.25) (layer F.Cu) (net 25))
 (segment (start 140.41 71.81) (end 138.0525 71.81) (width 0.25) (layer F.Cu) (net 25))
 (segment (start 137.9475 72.39) (end 137.9475 75.565) (width 0.25) (layer F.Cu) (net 25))
 (segment (start 131.2925 75.405) (end 131.2925 74.93) (width 0.25) (layer F.Cu) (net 24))
 (segment (start 131.1875 75.51) (end 131.2925 75.405) (width 0.25) (layer F.Cu) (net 24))
 (segment (start 128.83 75.51) (end 131.1875 75.51) (width 0.25) (layer F.Cu) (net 24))
 (segment (start 131.2925 74.93) (end 131.2925 72.39) (width 0.25) (layer F.Cu) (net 24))
 (segment (start 120.65 93.8275) (end 120.65 91.5925) (width 0.25) (layer F.Cu) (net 28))
 (segment (start 127.635 125.105) (end 127.645 125.095) (width 0.6) (layer F.Cu) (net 20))
 (segment (start 127.635 127.33) (end 127.635 125.105) (width 0.6) (layer F.Cu) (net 20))
 (segment (start 127.645 125.095) (end 127.645 123.18) (width 0.25) (layer F.Cu) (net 20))
 (segment (start 128.405 122.42) (end 129.54 122.42) (width 0.25) (layer F.Cu) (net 20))
 (segment (start 127.645 123.18) (end 128.405 122.42) (width 0.25) (layer F.Cu) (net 20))
 (segment (start 121.93 135.11) (end 122.555 134.485) (width 0.6) (layer F.Cu) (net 22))
 (segment (start 121.93 137.16) (end 121.93 135.11) (width 0.6) (layer F.Cu) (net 22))
 (segment (start 120.955 137.16) (end 120.015 136.22) (width 0.6) (layer F.Cu) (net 22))
 (segment (start 121.93 137.16) (end 120.955 137.16) (width 0.6) (layer F.Cu) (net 22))
 (segment (start 139.83 137.16) (end 142.145 137.16) (width 1) (layer F.Cu) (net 31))
 (segment (start 131.445 130.81) (end 134.69 130.81) (width 0.6) (layer F.Cu) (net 29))
 (segment (start 133.709174 137.16) (end 134.265 137.16) (width 1) (layer F.Cu) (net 29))
 (segment (start 131.41299 134.863816) (end 133.709174 137.16) (width 1) (layer F.Cu) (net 29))
 (segment (start 131.41299 132.090184) (end 131.41299 134.863816) (width 1) (layer F.Cu) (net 29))
 (segment (start 131.445 132.058174) (end 131.41299 132.090184) (width 1) (layer F.Cu) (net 29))
 (segment (start 131.445 130.81) (end 131.445 132.058174) (width 1) (layer F.Cu) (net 29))
 (segment (start 134.265 137.16) (end 137.03 137.16) (width 1) (layer F.Cu) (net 29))
 (segment (start 122.428001 117.601999) (end 123.19 116.84) (width 0.25) (layer F.Cu) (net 18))
 (segment (start 121.75499 118.27501) (end 122.428001 117.601999) (width 0.25) (layer F.Cu) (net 18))
 (segment (start 121.75499 128.14999) (end 121.75499 118.27501) (width 0.25) (layer F.Cu) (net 18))
 (segment (start 122.01 128.405) (end 121.75499 128.14999) (width 0.25) (layer F.Cu) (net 18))
 (segment (start 122.555 128.405) (end 122.01 128.405) (width 0.25) (layer F.Cu) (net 18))
 (segment (start 122.555 128.405) (end 122.555 125.73) (width 0.25) (layer F.Cu) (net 18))
 (segment (start 125.73 138.46) (end 125.73 137.16) (width 0.6) (layer F.Cu) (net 23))
 (segment (start 125.73 139.211523) (end 125.73 138.46) (width 0.6) (layer F.Cu) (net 23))
 (segment (start 128.19 141.671523) (end 125.73 139.211523) (width 0.6) (layer F.Cu) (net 23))
 (segment (start 128.19 143.51) (end 128.19 141.671523) (width 0.6) (layer F.Cu) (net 23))
 (segment (start 125.73 135.12) (end 125.095 134.485) (width 0.6) (layer F.Cu) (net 23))
 (segment (start 125.73 137.16) (end 125.73 135.12) (width 0.6) (layer F.Cu) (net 23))
 (segment (start 123.19 140.335) (end 120.015 137.795) (width 0.6) (layer F.Cu) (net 27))
 (segment (start 123.19 143.51) (end 123.19 140.335) (width 0.6) (layer F.Cu) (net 27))
 (segment (start 146.145 140.715) (end 143.35 143.51) (width 1) (layer F.Cu) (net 30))
 (segment (start 146.145 137.16) (end 146.145 140.715) (width 1) (layer F.Cu) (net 30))
 (segment (start 127.635 129.3425) (end 127.635 128.905) (width 0.6) (layer F.Cu) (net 32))
 (segment (start 127.635 137.985002) (end 127.635 129.3425) (width 0.6) (layer F.Cu) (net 32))
 (segment (start 129.990001 140.340003) (end 127.635 137.985002) (width 0.6) (layer F.Cu) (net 32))
 (segment (start 129.990001 144.374001) (end 129.990001 140.340003) (width 0.6) (layer F.Cu) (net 32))
 (segment (start 130.926001 145.310001) (end 129.990001 144.374001) (width 0.6) (layer F.Cu) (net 32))
 (segment (start 136.549999 145.310001) (end 130.926001 145.310001) (width 0.6) (layer F.Cu) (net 32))
 (segment (start 138.35 143.51) (end 136.549999 145.310001) (width 0.6) (layer F.Cu) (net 32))
 (segment (start 120.65 101.4475) (end 120.65 99.2125) (width 0.25) (layer F.Cu) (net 26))
 (segment (start 123.19 119.38) (end 125.5775 119.38) (width 0.25) (layer F.Cu) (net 19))
 (segment (start 128.995 116.34) (end 129.54 116.34) (width 0.25) (layer F.Cu) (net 19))
 (segment (start 128.1425 116.34) (end 128.995 116.34) (width 0.25) (layer F.Cu) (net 19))
 (segment (start 125.5775 118.905) (end 128.1425 116.34) (width 0.25) (layer F.Cu) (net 19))
 (segment (start 125.5775 119.38) (end 125.5775 118.905) (width 0.25) (layer F.Cu) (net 19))
 (segment (start 122.11237 104.14) (end 123.19 104.14) (width 0.25) (layer F.Cu) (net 13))
 (segment (start 121.33 104.14) (end 122.11237 104.14) (width 0.25) (layer F.Cu) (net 13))
 (segment (start 120.65 103.46) (end 121.33 104.14) (width 0.25) (layer F.Cu) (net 13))
 (segment (start 120.65 103.0225) (end 120.65 103.46) (width 0.25) (layer F.Cu) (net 13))
 (segment (start 141.935 132.08) (end 142.24 132.385) (width 0.6) (layer F.Cu) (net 35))
 (segment (start 139.63 132.08) (end 141.935 132.08) (width 0.6) (layer F.Cu) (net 35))
 (segment (start 142.24 132.385) (end 142.24 133.985) (width 0.6) (layer F.Cu) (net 35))
 (segment (start 146.05 132.8225) (end 146.05 132.385) (width 0.6) (layer F.Cu) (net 33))
 (segment (start 146.05 133.241482) (end 146.05 132.8225) (width 0.6) (layer F.Cu) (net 33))
 (segment (start 144.331472 134.96001) (end 146.05 133.241482) (width 0.6) (layer F.Cu) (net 33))
 (segment (start 140.34001 134.96001) (end 144.331472 134.96001) (width 0.6) (layer F.Cu) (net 33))
 (segment (start 139.63 134.25) (end 140.34001 134.96001) (width 0.6) (layer F.Cu) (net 33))
 (segment (start 139.63 133.35) (end 139.63 134.25) (width 0.6) (layer F.Cu) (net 33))
 (segment (start 146.525 129.0575) (end 146.05 129.0575) (width 0.6) (layer F.Cu) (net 33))
 (segment (start 147.02501 129.55751) (end 146.525 129.0575) (width 0.6) (layer F.Cu) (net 33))
 (segment (start 147.02501 131.88499) (end 147.02501 129.55751) (width 0.6) (layer F.Cu) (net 33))
 (segment (start 146.525 132.385) (end 147.02501 131.88499) (width 0.6) (layer F.Cu) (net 33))
 (segment (start 146.05 132.385) (end 146.525 132.385) (width 0.6) (layer F.Cu) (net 33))
 (segment (start 133.2485 133.35) (end 132.588 132.6895) (width 0.6) (layer F.Cu) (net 37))
 (segment (start 134.69 133.35) (end 133.2485 133.35) (width 0.6) (layer F.Cu) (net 37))
 (segment (start 143.6625 128.905) (end 144.78 128.905) (width 0.6) (layer F.Cu) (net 36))
 (segment (start 134.69 129.54) (end 134.62 129.54) (width 0.6) (layer F.Cu) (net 36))
 (segment (start 134.62 129.54) (end 133.35 128.27) (width 0.6) (layer F.Cu) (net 36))
 (via (at 144.78 128.905) (size 0.8) (drill 0.4) (layers F.Cu B.Cu) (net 36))
 (segment (start 133.35 128.27) (end 133.35 128.27) (width 0.6) (layer F.Cu) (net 36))
 (via (at 133.35 128.27) (size 0.8) (drill 0.4) (layers F.Cu B.Cu) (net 36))
 (segment (start 133.985 128.905) (end 133.35 128.27) (width 0.6) (layer B.Cu) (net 36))
 (segment (start 144.78 128.905) (end 133.985 128.905) (width 0.6) (layer B.Cu) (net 36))
 (segment (start 143.815 132.715) (end 144.145 132.385) (width 0.6) (layer F.Cu) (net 34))
 (segment (start 143.815 133.985) (end 143.815 132.715) (width 0.6) (layer F.Cu) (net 34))
 (via (at 137.16 130.81) (size 1.105) (drill 0.65) (layers F.Cu B.Cu) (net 2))
 (segment (start 139.63 130.81) (end 146.05 130.81) (width 0.6) (layer F.Cu) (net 2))
 (segment (start 122.11237 96.52) (end 123.19 96.52) (width 0.25) (layer F.Cu) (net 2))
 (segment (start 121.33 96.52) (end 122.11237 96.52) (width 0.25) (layer F.Cu) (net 2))
 (segment (start 120.65 97.2) (end 121.33 96.52) (width 0.25) (layer F.Cu) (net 2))
 (segment (start 120.65 97.6375) (end 120.65 97.2) (width 0.25) (layer F.Cu) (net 2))
 (segment (start 120.65 95.84) (end 121.33 96.52) (width 0.25) (layer F.Cu) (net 2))
 (segment (start 120.65 95.4025) (end 120.65 95.84) (width 0.25) (layer F.Cu) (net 2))
 (via (at 137.16 132.715) (size 1.105) (drill 0.65) (layers F.Cu B.Cu) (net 2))
 (via (at 137.16 134.62) (size 1.105) (drill 0.65) (layers F.Cu B.Cu) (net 2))
 (via (at 139.065 135.255) (size 1.105) (drill 0.65) (layers F.Cu B.Cu) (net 2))
 (via (at 135.255 134.62) (size 1.105) (drill 0.65) (layers F.Cu B.Cu) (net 2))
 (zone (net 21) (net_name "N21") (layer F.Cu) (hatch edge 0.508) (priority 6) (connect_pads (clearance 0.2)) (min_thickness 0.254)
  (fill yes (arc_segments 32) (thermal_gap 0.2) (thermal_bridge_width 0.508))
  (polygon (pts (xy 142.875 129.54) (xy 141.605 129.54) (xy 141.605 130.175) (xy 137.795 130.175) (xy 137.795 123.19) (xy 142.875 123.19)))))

